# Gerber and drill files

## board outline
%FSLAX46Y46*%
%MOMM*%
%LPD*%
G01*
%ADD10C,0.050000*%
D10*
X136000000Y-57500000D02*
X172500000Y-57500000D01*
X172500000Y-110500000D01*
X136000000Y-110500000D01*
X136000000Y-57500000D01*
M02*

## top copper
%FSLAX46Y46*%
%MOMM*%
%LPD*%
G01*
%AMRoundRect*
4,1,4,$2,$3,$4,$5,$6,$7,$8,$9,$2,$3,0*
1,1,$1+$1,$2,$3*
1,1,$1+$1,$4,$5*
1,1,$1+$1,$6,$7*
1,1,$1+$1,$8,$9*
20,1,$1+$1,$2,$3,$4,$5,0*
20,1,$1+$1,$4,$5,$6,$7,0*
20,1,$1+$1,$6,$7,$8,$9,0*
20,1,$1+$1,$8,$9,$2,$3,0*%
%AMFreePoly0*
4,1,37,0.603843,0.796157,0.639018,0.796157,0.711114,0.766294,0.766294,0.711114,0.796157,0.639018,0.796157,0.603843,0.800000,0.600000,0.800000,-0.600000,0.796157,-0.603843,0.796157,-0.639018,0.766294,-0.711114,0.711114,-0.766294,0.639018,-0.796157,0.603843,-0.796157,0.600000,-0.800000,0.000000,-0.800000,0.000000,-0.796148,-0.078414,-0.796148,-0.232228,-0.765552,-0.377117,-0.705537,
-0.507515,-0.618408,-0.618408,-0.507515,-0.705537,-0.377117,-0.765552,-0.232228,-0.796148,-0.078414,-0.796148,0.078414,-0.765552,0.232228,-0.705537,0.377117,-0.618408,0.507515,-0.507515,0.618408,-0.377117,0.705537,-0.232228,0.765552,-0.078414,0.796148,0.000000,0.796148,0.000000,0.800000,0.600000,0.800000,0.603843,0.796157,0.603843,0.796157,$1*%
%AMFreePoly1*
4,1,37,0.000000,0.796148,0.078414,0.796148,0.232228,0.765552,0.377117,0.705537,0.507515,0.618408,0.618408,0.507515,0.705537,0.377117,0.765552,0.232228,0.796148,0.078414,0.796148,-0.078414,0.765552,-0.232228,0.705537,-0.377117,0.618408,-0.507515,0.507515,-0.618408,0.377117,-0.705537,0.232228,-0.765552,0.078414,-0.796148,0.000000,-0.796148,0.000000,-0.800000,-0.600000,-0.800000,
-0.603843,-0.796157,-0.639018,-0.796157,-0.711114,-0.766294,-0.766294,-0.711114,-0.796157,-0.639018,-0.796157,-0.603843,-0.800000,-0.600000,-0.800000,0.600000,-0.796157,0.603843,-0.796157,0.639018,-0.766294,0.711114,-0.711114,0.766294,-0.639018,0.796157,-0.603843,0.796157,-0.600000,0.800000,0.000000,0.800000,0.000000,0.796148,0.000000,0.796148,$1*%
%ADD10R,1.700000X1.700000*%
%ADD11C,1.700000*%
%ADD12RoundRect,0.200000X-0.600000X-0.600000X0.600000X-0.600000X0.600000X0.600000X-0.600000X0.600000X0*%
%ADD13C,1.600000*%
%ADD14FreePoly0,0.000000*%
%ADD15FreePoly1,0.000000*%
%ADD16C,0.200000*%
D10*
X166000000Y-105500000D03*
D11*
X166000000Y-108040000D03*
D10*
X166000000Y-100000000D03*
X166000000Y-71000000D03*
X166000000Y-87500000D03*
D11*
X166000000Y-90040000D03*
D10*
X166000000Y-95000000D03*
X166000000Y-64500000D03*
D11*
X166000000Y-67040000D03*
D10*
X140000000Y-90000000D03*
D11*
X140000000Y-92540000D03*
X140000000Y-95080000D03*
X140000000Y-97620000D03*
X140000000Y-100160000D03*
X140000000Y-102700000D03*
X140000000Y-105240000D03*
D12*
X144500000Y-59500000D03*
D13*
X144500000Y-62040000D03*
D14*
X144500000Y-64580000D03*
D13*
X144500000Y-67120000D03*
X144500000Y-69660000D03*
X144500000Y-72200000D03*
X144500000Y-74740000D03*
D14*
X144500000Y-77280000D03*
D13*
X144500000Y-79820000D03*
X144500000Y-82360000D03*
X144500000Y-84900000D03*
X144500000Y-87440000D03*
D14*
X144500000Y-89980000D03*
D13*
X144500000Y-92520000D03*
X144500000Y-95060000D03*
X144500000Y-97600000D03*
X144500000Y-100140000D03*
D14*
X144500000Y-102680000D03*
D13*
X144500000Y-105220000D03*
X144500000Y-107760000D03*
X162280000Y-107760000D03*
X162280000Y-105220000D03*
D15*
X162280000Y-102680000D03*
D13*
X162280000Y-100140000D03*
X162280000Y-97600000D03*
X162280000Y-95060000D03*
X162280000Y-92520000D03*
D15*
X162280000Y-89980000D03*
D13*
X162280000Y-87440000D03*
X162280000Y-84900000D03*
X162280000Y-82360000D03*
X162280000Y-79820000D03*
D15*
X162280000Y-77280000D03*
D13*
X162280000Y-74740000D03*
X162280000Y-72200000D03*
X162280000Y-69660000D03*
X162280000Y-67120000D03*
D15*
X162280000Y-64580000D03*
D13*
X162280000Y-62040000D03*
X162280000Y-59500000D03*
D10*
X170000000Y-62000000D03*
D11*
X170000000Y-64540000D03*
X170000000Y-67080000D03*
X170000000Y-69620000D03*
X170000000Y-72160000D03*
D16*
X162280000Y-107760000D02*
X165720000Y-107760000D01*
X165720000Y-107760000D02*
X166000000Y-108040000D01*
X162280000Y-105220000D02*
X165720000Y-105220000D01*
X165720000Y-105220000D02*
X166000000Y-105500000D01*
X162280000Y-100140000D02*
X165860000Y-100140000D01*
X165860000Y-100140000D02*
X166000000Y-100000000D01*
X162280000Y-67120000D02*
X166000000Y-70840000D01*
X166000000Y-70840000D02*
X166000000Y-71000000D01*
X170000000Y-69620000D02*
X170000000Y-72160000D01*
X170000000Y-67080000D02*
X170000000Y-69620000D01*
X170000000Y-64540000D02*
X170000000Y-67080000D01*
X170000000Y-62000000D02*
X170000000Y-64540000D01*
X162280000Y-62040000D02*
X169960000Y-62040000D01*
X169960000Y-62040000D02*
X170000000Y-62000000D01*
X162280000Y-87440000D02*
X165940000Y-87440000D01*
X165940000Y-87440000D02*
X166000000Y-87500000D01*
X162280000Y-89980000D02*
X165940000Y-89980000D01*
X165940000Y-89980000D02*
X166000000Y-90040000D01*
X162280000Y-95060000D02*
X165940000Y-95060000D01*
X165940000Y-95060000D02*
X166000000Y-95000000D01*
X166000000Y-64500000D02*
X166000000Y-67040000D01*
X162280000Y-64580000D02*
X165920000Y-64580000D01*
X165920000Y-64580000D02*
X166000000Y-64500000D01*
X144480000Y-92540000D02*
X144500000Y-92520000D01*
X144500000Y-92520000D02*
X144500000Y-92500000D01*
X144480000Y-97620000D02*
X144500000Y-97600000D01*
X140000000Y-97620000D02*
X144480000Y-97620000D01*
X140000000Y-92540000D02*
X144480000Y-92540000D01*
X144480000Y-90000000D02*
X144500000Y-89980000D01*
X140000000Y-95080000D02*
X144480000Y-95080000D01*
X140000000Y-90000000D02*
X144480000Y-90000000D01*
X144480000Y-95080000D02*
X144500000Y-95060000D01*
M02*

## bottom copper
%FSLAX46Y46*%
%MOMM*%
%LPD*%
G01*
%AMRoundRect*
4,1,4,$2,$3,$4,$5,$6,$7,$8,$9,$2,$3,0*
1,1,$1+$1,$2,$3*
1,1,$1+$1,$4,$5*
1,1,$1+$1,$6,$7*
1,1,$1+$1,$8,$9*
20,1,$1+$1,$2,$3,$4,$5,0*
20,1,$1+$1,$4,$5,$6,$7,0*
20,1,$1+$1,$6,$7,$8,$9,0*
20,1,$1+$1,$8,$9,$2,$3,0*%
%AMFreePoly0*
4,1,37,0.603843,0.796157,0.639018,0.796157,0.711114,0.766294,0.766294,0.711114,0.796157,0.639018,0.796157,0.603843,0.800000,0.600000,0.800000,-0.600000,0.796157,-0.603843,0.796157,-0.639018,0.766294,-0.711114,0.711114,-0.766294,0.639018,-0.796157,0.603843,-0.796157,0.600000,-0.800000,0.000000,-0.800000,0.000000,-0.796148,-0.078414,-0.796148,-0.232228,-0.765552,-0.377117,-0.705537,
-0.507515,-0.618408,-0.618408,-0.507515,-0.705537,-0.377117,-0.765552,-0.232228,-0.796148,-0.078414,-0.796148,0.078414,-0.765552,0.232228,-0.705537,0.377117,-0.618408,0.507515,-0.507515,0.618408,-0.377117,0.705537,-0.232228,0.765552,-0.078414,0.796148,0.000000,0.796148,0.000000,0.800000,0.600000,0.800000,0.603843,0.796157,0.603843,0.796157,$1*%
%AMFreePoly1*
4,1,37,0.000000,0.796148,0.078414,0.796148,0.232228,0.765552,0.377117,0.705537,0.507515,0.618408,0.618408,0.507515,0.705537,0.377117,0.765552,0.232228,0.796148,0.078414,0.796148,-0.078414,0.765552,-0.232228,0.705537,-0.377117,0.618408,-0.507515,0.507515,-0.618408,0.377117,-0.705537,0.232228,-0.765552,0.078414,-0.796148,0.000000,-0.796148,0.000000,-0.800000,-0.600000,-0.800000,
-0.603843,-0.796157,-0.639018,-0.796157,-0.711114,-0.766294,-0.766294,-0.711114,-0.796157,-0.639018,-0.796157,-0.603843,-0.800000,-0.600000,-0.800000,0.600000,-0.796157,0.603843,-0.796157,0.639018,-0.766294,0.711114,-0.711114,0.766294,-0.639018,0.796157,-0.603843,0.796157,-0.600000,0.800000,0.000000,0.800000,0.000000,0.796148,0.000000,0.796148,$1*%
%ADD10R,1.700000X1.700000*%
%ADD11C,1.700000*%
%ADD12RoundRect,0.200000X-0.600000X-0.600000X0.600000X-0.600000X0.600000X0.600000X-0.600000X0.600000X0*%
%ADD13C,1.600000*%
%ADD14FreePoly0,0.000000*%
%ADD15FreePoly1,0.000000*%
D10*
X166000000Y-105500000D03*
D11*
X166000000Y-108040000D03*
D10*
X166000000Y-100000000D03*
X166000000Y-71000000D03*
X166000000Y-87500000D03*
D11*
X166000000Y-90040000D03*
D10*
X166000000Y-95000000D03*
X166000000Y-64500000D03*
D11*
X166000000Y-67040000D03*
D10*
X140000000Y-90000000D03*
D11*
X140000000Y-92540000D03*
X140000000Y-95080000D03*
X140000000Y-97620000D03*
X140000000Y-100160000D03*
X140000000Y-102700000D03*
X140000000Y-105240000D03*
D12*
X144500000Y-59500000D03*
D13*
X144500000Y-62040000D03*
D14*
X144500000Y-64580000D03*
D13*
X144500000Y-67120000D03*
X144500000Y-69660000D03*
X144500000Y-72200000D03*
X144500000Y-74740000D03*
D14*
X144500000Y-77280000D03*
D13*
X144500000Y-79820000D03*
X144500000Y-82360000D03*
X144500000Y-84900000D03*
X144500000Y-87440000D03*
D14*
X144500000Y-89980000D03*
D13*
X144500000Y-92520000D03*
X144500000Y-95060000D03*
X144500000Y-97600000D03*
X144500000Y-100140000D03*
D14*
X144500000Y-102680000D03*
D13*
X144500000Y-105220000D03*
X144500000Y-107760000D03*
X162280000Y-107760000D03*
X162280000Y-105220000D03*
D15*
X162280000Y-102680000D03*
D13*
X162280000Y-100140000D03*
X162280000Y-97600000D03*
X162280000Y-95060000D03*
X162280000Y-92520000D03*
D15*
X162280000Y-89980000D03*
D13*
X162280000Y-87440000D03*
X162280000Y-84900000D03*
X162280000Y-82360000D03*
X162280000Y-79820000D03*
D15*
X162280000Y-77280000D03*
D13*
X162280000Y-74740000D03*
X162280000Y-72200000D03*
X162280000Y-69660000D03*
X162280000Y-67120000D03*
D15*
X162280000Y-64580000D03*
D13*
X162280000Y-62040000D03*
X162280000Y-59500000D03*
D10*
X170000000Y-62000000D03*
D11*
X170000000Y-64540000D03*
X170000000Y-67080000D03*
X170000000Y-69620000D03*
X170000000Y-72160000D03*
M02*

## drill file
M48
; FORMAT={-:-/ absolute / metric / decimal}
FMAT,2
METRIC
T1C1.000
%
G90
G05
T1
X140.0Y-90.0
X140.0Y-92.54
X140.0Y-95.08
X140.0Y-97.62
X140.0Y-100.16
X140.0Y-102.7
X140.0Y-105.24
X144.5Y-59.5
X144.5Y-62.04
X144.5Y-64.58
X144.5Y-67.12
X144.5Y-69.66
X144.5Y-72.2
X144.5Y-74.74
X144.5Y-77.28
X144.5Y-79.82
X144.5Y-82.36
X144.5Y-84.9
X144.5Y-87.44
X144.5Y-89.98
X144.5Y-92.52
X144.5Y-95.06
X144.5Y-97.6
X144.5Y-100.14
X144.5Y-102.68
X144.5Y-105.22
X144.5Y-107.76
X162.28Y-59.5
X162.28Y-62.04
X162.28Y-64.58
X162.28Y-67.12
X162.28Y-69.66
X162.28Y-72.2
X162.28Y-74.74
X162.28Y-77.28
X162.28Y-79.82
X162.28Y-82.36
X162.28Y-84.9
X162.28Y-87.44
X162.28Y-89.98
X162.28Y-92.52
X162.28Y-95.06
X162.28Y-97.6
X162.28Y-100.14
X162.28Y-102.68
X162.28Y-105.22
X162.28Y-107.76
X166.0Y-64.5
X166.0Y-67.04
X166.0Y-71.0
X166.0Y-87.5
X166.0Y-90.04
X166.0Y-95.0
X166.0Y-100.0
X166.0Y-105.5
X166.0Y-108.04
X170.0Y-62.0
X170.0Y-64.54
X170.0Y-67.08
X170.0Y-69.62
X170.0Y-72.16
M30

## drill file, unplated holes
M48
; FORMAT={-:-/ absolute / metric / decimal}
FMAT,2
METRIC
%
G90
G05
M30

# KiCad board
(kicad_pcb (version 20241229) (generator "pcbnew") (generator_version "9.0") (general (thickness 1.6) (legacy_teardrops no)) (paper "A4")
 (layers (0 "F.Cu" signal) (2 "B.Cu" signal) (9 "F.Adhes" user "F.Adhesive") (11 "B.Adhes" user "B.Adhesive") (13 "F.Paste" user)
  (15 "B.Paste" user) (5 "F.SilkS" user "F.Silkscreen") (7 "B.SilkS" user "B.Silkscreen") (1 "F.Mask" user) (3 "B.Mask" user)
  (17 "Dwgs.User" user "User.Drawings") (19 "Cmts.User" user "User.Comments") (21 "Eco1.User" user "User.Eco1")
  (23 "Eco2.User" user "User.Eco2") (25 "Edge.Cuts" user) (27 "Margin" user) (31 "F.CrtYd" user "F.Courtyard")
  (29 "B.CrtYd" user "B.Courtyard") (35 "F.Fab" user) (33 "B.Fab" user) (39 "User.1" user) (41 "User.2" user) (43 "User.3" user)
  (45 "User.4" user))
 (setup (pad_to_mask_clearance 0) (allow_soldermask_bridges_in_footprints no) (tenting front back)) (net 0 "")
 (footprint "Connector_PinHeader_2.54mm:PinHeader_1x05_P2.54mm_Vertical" (layer "F.Cu") (at 170 62)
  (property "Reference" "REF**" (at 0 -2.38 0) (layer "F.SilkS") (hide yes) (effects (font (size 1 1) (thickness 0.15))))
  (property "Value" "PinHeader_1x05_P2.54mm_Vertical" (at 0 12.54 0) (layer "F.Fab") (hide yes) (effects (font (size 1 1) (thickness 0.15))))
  (pad "1" thru_hole rect (at 0 0) (size 1.7 1.7) (drill 1) (layers "*.Cu" "*.Mask") (remove_unused_layers no))
  (pad "2" thru_hole circle (at 0 2.54) (size 1.7 1.7) (drill 1) (layers "*.Cu" "*.Mask") (remove_unused_layers no))
  (pad "3" thru_hole circle (at 0 5.08) (size 1.7 1.7) (drill 1) (layers "*.Cu" "*.Mask") (remove_unused_layers no))
  (pad "4" thru_hole circle (at 0 7.62) (size 1.7 1.7) (drill 1) (layers "*.Cu" "*.Mask") (remove_unused_layers no))
  (pad "5" thru_hole circle (at 0 10.16) (size 1.7 1.7) (drill 1) (layers "*.Cu" "*.Mask") (remove_unused_layers no)))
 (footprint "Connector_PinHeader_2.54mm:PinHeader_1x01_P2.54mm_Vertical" (layer "F.Cu") (at 166 71)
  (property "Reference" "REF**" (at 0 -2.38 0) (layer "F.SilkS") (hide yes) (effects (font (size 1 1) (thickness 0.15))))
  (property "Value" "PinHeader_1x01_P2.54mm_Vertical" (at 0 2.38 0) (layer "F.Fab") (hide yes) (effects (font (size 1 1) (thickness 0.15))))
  (pad "1" thru_hole rect (at 0 0) (size 1.7 1.7) (drill 1) (layers "*.Cu" "*.Mask") (remove_unused_layers no)))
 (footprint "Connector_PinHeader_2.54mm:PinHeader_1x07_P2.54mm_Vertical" (layer "F.Cu") (at 140 90)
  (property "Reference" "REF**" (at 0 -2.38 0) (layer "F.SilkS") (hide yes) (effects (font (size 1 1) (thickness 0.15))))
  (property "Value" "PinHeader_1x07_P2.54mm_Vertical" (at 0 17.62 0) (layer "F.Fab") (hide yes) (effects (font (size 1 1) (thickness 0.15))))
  (pad "1" thru_hole rect (at 0 0) (size 1.7 1.7) (drill 1) (layers "*.Cu" "*.Mask") (remove_unused_layers no))
  (pad "2" thru_hole circle (at 0 2.54) (size 1.7 1.7) (drill 1) (layers "*.Cu" "*.Mask") (remove_unused_layers no))
  (pad "3" thru_hole circle (at 0 5.08) (size 1.7 1.7) (drill 1) (layers "*.Cu" "*.Mask") (remove_unused_layers no))
  (pad "4" thru_hole circle (at 0 7.62) (size 1.7 1.7) (drill 1) (layers "*.Cu" "*.Mask") (remove_unused_layers no))
  (pad "5" thru_hole circle (at 0 10.16) (size 1.7 1.7) (drill 1) (layers "*.Cu" "*.Mask") (remove_unused_layers no))
  (pad "6" thru_hole circle (at 0 12.7) (size 1.7 1.7) (drill 1) (layers "*.Cu" "*.Mask") (remove_unused_layers no))
  (pad "7" thru_hole circle (at 0 15.24) (size 1.7 1.7) (drill 1) (layers "*.Cu" "*.Mask") (remove_unused_layers no)))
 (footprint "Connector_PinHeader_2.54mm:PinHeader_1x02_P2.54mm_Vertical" (layer "F.Cu") (at 166 87.5)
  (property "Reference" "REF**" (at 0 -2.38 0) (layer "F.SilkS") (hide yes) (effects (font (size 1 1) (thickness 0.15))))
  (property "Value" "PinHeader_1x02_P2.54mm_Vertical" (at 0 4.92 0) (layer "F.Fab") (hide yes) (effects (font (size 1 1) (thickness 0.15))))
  (pad "1" thru_hole rect (at 0 0) (size 1.7 1.7) (drill 1) (layers "*.Cu" "*.Mask") (remove_unused_layers no))
  (pad "2" thru_hole circle (at 0 2.54) (size 1.7 1.7) (drill 1) (layers "*.Cu" "*.Mask") (remove_unused_layers no)))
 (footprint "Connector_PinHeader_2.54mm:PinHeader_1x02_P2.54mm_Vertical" (layer "F.Cu") (at 166 64.5)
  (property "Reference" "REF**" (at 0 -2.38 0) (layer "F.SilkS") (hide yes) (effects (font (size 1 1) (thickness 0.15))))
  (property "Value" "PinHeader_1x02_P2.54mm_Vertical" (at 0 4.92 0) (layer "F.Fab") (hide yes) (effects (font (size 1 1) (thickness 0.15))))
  (pad "1" thru_hole rect (at 0 0) (size 1.7 1.7) (drill 1) (layers "*.Cu" "*.Mask") (remove_unused_layers no))
  (pad "2" thru_hole circle (at 0 2.54) (size 1.7 1.7) (drill 1) (layers "*.Cu" "*.Mask") (remove_unused_layers no)))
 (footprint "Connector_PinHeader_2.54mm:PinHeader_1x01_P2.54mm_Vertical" (layer "F.Cu") (at 166 100)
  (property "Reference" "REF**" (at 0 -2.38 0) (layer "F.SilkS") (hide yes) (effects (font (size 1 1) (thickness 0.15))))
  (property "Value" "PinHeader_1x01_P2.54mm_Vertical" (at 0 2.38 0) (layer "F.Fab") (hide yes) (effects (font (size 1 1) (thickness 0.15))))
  (pad "1" thru_hole rect (at 0 0) (size 1.7 1.7) (drill 1) (layers "*.Cu" "*.Mask") (remove_unused_layers no)))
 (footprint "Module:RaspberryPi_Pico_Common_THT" (layer "F.Cu") (at 144.5 59.5)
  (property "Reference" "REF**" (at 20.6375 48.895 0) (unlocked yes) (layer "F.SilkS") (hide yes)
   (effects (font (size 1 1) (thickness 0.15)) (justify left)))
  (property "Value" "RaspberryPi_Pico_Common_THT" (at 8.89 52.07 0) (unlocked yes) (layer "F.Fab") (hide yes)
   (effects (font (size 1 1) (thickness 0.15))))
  (pad "1" thru_hole roundrect (at 0 0) (size 1.6 1.6) (drill 1) (layers "*.Cu" "*.Mask") (remove_unused_layers no) (roundrect_rratio 0.125))
  (pad "2" thru_hole circle (at 0 2.54) (size 1.6 1.6) (drill 1) (layers "*.Cu" "*.Mask") (remove_unused_layers no))
  (pad "3" thru_hole custom (at 0 5.08) (size 1.6 1.6) (drill 1) (layers "*.Cu" "*.Mask") (remove_unused_layers no)
   (options (clearance outline) (anchor circle)) (primitives))
  (pad "4" thru_hole circle (at 0 7.62) (size 1.6 1.6) (drill 1) (layers "*.Cu" "*.Mask") (remove_unused_layers no))
  (pad "5" thru_hole circle (at 0 10.16) (size 1.6 1.6) (drill 1) (layers "*.Cu" "*.Mask") (remove_unused_layers no))
  (pad "6" thru_hole circle (at 0 12.7) (size 1.6 1.6) (drill 1) (layers "*.Cu" "*.Mask") (remove_unused_layers no))
  (pad "7" thru_hole circle (at 0 15.24) (size 1.6 1.6) (drill 1) (layers "*.Cu" "*.Mask") (remove_unused_layers no))
  (pad "8" thru_hole custom (at 0 17.78) (size 1.6 1.6) (drill 1) (layers "*.Cu" "*.Mask") (remove_unused_layers no)
   (options (clearance outline) (anchor circle)) (primitives))
  (pad "9" thru_hole circle (at 0 20.32) (size 1.6 1.6) (drill 1) (layers "*.Cu" "*.Mask") (remove_unused_layers no))
  (pad "10" thru_hole circle (at 0 22.86) (size 1.6 1.6) (drill 1) (layers "*.Cu" "*.Mask") (remove_unused_layers no))
  (pad "11" thru_hole circle (at 0 25.4) (size 1.6 1.6) (drill 1) (layers "*.Cu" "*.Mask") (remove_unused_layers no))
  (pad "12" thru_hole circle (at 0 27.94) (size 1.6 1.6) (drill 1) (layers "*.Cu" "*.Mask") (remove_unused_layers no))
  (pad "13" thru_hole custom (at 0 30.48) (size 1.6 1.6) (drill 1) (layers "*.Cu" "*.Mask") (remove_unused_layers no)
   (options (clearance outline) (anchor circle)) (primitives))
  (pad "14" thru_hole circle (at 0 33.02) (size 1.6 1.6) (drill 1) (layers "*.Cu" "*.Mask") (remove_unused_layers no))
  (pad "15" thru_hole circle (at 0 35.56) (size 1.6 1.6) (drill 1) (layers "*.Cu" "*.Mask") (remove_unused_layers no))
  (pad "16" thru_hole circle (at 0 38.1) (size 1.6 1.6) (drill 1) (layers "*.Cu" "*.Mask") (remove_unused_layers no))
  (pad "17" thru_hole circle (at 0 40.64) (size 1.6 1.6) (drill 1) (layers "*.Cu" "*.Mask") (remove_unused_layers no))
  (pad "18" thru_hole custom (at 0 43.18) (size 1.6 1.6) (drill 1) (layers "*.Cu" "*.Mask") (remove_unused_layers no)
   (options (clearance outline) (anchor circle)) (primitives))
  (pad "19" thru_hole circle (at 0 45.72) (size 1.6 1.6) (drill 1) (layers "*.Cu" "*.Mask") (remove_unused_layers no))
  (pad "20" thru_hole circle (at 0 48.26) (size 1.6 1.6) (drill 1) (layers "*.Cu" "*.Mask") (remove_unused_layers no))
  (pad "21" thru_hole circle (at 17.78 48.26) (size 1.6 1.6) (drill 1) (layers "*.Cu" "*.Mask") (remove_unused_layers no))
  (pad "22" thru_hole circle (at 17.78 45.72) (size 1.6 1.6) (drill 1) (layers "*.Cu" "*.Mask") (remove_unused_layers no))
  (pad "23" thru_hole custom (at 17.78 43.18) (size 1.6 1.6) (drill 1) (layers "*.Cu" "*.Mask") (remove_unused_layers no)
   (options (clearance outline) (anchor circle)) (primitives))
  (pad "24" thru_hole circle (at 17.78 40.64) (size 1.6 1.6) (drill 1) (layers "*.Cu" "*.Mask") (remove_unused_layers no))
  (pad "25" thru_hole circle (at 17.78 38.1) (size 1.6 1.6) (drill 1) (layers "*.Cu" "*.Mask") (remove_unused_layers no))
  (pad "26" thru_hole circle (at 17.78 35.56) (size 1.6 1.6) (drill 1) (layers "*.Cu" "*.Mask") (remove_unused_layers no))
  (pad "27" thru_hole circle (at 17.78 33.02) (size 1.6 1.6) (drill 1) (layers "*.Cu" "*.Mask") (remove_unused_layers no))
  (pad "28" thru_hole custom (at 17.78 30.48) (size 1.6 1.6) (drill 1) (layers "*.Cu" "*.Mask") (remove_unused_layers no)
   (options (clearance outline) (anchor circle)) (primitives))
  (pad "29" thru_hole circle (at 17.78 27.94) (size 1.6 1.6) (drill 1) (layers "*.Cu" "*.Mask") (remove_unused_layers no))
  (pad "30" thru_hole circle (at 17.78 25.4) (size 1.6 1.6) (drill 1) (layers "*.Cu" "*.Mask") (remove_unused_layers no))
  (pad "31" thru_hole circle (at 17.78 22.86) (size 1.6 1.6) (drill 1) (layers "*.Cu" "*.Mask") (remove_unused_layers no))
  (pad "32" thru_hole circle (at 17.78 20.32) (size 1.6 1.6) (drill 1) (layers "*.Cu" "*.Mask") (remove_unused_layers no))
  (pad "33" thru_hole custom (at 17.78 17.78) (size 1.6 1.6) (drill 1) (layers "*.Cu" "*.Mask") (remove_unused_layers no)
   (options (clearance outline) (anchor circle)) (primitives))
  (pad "34" thru_hole circle (at 17.78 15.24) (size 1.6 1.6) (drill 1) (layers "*.Cu" "*.Mask") (remove_unused_layers no))
  (pad "35" thru_hole circle (at 17.78 12.7) (size 1.6 1.6) (drill 1) (layers "*.Cu" "*.Mask") (remove_unused_layers no))
  (pad "36" thru_hole circle (at 17.78 10.16) (size 1.6 1.6) (drill 1) (layers "*.Cu" "*.Mask") (remove_unused_layers no))
  (pad "37" thru_hole circle (at 17.78 7.62) (size 1.6 1.6) (drill 1) (layers "*.Cu" "*.Mask") (remove_unused_layers no))
  (pad "38" thru_hole custom (at 17.78 5.08) (size 1.6 1.6) (drill 1) (layers "*.Cu" "*.Mask") (remove_unused_layers no)
   (options (clearance outline) (anchor circle)) (primitives))
  (pad "39" thru_hole circle (at 17.78 2.54) (size 1.6 1.6) (drill 1) (layers "*.Cu" "*.Mask") (remove_unused_layers no))
  (pad "40" thru_hole circle (at 17.78 0) (size 1.6 1.6) (drill 1) (layers "*.Cu" "*.Mask") (remove_unused_layers no)))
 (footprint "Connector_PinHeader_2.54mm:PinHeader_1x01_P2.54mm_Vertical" (layer "F.Cu") (at 166 95)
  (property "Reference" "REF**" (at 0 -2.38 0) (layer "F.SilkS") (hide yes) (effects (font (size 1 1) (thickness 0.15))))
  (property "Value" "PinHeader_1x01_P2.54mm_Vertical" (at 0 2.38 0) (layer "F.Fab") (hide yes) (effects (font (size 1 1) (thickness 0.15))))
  (pad "1" thru_hole rect (at 0 0) (size 1.7 1.7) (drill 1) (layers "*.Cu" "*.Mask") (remove_unused_layers no)))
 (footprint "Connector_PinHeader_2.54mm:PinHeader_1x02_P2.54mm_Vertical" (layer "F.Cu") (at 166 105.5)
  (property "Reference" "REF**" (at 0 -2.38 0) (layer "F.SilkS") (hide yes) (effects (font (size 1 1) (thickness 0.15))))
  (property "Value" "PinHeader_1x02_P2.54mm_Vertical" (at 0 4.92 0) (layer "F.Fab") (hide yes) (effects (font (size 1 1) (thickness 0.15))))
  (pad "1" thru_hole rect (at 0 0) (size 1.7 1.7) (drill 1) (layers "*.Cu" "*.Mask") (remove_unused_layers no))
  (pad "2" thru_hole circle (at 0 2.54) (size 1.7 1.7) (drill 1) (layers "*.Cu" "*.Mask") (remove_unused_layers no)))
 (gr_rect (start 136 57.5) (end 172.5 110.5) (stroke (width 0.05) (type default)) (fill no) (layer "Edge.Cuts"))
 (segment (start 165.72 105.22) (end 166 105.5) (width 0.2) (layer "F.Cu") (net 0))
 (segment (start 165.94 89.98) (end 166 90.04) (width 0.2) (layer "F.Cu") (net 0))
 (segment (start 140.02 105.22) (end 140 105.24) (width 0.2) (layer "F.Cu") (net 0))
 (segment (start 162.28 95.06) (end 165.94 95.06) (width 0.2) (layer "F.Cu") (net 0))
 (segment (start 166 70.84) (end 166 71) (width 0.2) (layer "F.Cu") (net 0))
 (segment (start 144.5 100.14) (end 140.02 100.14) (width 0.2) (layer "F.Cu") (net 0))
 (segment (start 144.48 92.54) (end 144.5 92.52) (width 0.2) (layer "F.Cu") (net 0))
 (segment (start 166 64.5) (end 166 67.04) (width 0.2) (layer "F.Cu") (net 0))
 (segment (start 162.28 105.22) (end 165.72 105.22) (width 0.2) (layer "F.Cu") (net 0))
 (segment (start 162.28 87.44) (end 165.94 87.44) (width 0.2) (layer "F.Cu") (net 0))
 (segment (start 144.5 92.52) (end 144.5 92.5) (width 0.2) (layer "F.Cu") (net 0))
 (segment (start 165.72 107.76) (end 166 108.04) (width 0.2) (layer "F.Cu") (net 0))
 (segment (start 162.28 67.12) (end 166 70.84) (width 0.2) (layer "F.Cu") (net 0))
 (segment (start 165.94 95.06) (end 166 95) (width 0.2) (layer "F.Cu") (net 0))
 (segment (start 165.94 87.44) (end 166 87.5) (width 0.2) (layer "F.Cu") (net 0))
 (segment (start 140.02 100.14) (end 140 100.16) (width 0.2) (layer "F.Cu") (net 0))
 (segment (start 170 69.62) (end 170 72.16) (width 0.2) (layer "F.Cu") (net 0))
 (segment (start 170 62) (end 170 64.54) (width 0.2) (layer "F.Cu") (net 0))
 (segment (start 162.28 62.04) (end 169.96 62.04) (width 0.2) (layer "F.Cu") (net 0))
 (segment (start 170 64.54) (end 170 67.08) (width 0.2) (layer "F.Cu") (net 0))
 (segment (start 144.48 97.62) (end 144.5 97.6) (width 0.2) (layer "F.Cu") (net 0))
 (segment (start 140 97.62) (end 144.48 97.62) (width 0.2) (layer "F.Cu") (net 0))
 (segment (start 170 67.08) (end 170 69.62) (width 0.2) (layer "F.Cu") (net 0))
 (segment (start 162.28 107.76) (end 165.72 107.76) (width 0.2) (layer "F.Cu") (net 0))
 (segment (start 144.5 105.22) (end 140.02 105.22) (width 0.2) (layer "F.Cu") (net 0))
 (segment (start 144.5 102.68) (end 140.02 102.68) (width 0.2) (layer "F.Cu") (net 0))
 (segment (start 140 92.54) (end 144.48 92.54) (width 0.2) (layer "F.Cu") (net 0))
 (segment (start 140.02 102.68) (end 140 102.7) (width 0.2) (layer "F.Cu") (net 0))
 (segment (start 162.28 100.14) (end 165.86 100.14) (width 0.2) (layer "F.Cu") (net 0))
 (segment (start 144.48 90) (end 144.5 89.98) (width 0.2) (layer "F.Cu") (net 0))
 (segment (start 162.28 64.58) (end 165.92 64.58) (width 0.2) (layer "F.Cu") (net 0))
 (segment (start 140 95.08) (end 144.48 95.08) (width 0.2) (layer "F.Cu") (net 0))
 (segment (start 169.96 62.04) (end 170 62) (width 0.2) (layer "F.Cu") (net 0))
 (segment (start 140 90) (end 144.48 90) (width 0.2) (layer "F.Cu") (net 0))
 (segment (start 165.92 64.58) (end 166 64.5) (width 0.2) (layer "F.Cu") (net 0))
 (segment (start 165.86 100.14) (end 166 100) (width 0.2) (layer "F.Cu") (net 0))
 (segment (start 162.28 89.98) (end 165.94 89.98) (width 0.2) (layer "F.Cu") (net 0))
 (segment (start 144.48 95.08) (end 144.5 95.06) (width 0.2) (layer "F.Cu") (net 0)))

